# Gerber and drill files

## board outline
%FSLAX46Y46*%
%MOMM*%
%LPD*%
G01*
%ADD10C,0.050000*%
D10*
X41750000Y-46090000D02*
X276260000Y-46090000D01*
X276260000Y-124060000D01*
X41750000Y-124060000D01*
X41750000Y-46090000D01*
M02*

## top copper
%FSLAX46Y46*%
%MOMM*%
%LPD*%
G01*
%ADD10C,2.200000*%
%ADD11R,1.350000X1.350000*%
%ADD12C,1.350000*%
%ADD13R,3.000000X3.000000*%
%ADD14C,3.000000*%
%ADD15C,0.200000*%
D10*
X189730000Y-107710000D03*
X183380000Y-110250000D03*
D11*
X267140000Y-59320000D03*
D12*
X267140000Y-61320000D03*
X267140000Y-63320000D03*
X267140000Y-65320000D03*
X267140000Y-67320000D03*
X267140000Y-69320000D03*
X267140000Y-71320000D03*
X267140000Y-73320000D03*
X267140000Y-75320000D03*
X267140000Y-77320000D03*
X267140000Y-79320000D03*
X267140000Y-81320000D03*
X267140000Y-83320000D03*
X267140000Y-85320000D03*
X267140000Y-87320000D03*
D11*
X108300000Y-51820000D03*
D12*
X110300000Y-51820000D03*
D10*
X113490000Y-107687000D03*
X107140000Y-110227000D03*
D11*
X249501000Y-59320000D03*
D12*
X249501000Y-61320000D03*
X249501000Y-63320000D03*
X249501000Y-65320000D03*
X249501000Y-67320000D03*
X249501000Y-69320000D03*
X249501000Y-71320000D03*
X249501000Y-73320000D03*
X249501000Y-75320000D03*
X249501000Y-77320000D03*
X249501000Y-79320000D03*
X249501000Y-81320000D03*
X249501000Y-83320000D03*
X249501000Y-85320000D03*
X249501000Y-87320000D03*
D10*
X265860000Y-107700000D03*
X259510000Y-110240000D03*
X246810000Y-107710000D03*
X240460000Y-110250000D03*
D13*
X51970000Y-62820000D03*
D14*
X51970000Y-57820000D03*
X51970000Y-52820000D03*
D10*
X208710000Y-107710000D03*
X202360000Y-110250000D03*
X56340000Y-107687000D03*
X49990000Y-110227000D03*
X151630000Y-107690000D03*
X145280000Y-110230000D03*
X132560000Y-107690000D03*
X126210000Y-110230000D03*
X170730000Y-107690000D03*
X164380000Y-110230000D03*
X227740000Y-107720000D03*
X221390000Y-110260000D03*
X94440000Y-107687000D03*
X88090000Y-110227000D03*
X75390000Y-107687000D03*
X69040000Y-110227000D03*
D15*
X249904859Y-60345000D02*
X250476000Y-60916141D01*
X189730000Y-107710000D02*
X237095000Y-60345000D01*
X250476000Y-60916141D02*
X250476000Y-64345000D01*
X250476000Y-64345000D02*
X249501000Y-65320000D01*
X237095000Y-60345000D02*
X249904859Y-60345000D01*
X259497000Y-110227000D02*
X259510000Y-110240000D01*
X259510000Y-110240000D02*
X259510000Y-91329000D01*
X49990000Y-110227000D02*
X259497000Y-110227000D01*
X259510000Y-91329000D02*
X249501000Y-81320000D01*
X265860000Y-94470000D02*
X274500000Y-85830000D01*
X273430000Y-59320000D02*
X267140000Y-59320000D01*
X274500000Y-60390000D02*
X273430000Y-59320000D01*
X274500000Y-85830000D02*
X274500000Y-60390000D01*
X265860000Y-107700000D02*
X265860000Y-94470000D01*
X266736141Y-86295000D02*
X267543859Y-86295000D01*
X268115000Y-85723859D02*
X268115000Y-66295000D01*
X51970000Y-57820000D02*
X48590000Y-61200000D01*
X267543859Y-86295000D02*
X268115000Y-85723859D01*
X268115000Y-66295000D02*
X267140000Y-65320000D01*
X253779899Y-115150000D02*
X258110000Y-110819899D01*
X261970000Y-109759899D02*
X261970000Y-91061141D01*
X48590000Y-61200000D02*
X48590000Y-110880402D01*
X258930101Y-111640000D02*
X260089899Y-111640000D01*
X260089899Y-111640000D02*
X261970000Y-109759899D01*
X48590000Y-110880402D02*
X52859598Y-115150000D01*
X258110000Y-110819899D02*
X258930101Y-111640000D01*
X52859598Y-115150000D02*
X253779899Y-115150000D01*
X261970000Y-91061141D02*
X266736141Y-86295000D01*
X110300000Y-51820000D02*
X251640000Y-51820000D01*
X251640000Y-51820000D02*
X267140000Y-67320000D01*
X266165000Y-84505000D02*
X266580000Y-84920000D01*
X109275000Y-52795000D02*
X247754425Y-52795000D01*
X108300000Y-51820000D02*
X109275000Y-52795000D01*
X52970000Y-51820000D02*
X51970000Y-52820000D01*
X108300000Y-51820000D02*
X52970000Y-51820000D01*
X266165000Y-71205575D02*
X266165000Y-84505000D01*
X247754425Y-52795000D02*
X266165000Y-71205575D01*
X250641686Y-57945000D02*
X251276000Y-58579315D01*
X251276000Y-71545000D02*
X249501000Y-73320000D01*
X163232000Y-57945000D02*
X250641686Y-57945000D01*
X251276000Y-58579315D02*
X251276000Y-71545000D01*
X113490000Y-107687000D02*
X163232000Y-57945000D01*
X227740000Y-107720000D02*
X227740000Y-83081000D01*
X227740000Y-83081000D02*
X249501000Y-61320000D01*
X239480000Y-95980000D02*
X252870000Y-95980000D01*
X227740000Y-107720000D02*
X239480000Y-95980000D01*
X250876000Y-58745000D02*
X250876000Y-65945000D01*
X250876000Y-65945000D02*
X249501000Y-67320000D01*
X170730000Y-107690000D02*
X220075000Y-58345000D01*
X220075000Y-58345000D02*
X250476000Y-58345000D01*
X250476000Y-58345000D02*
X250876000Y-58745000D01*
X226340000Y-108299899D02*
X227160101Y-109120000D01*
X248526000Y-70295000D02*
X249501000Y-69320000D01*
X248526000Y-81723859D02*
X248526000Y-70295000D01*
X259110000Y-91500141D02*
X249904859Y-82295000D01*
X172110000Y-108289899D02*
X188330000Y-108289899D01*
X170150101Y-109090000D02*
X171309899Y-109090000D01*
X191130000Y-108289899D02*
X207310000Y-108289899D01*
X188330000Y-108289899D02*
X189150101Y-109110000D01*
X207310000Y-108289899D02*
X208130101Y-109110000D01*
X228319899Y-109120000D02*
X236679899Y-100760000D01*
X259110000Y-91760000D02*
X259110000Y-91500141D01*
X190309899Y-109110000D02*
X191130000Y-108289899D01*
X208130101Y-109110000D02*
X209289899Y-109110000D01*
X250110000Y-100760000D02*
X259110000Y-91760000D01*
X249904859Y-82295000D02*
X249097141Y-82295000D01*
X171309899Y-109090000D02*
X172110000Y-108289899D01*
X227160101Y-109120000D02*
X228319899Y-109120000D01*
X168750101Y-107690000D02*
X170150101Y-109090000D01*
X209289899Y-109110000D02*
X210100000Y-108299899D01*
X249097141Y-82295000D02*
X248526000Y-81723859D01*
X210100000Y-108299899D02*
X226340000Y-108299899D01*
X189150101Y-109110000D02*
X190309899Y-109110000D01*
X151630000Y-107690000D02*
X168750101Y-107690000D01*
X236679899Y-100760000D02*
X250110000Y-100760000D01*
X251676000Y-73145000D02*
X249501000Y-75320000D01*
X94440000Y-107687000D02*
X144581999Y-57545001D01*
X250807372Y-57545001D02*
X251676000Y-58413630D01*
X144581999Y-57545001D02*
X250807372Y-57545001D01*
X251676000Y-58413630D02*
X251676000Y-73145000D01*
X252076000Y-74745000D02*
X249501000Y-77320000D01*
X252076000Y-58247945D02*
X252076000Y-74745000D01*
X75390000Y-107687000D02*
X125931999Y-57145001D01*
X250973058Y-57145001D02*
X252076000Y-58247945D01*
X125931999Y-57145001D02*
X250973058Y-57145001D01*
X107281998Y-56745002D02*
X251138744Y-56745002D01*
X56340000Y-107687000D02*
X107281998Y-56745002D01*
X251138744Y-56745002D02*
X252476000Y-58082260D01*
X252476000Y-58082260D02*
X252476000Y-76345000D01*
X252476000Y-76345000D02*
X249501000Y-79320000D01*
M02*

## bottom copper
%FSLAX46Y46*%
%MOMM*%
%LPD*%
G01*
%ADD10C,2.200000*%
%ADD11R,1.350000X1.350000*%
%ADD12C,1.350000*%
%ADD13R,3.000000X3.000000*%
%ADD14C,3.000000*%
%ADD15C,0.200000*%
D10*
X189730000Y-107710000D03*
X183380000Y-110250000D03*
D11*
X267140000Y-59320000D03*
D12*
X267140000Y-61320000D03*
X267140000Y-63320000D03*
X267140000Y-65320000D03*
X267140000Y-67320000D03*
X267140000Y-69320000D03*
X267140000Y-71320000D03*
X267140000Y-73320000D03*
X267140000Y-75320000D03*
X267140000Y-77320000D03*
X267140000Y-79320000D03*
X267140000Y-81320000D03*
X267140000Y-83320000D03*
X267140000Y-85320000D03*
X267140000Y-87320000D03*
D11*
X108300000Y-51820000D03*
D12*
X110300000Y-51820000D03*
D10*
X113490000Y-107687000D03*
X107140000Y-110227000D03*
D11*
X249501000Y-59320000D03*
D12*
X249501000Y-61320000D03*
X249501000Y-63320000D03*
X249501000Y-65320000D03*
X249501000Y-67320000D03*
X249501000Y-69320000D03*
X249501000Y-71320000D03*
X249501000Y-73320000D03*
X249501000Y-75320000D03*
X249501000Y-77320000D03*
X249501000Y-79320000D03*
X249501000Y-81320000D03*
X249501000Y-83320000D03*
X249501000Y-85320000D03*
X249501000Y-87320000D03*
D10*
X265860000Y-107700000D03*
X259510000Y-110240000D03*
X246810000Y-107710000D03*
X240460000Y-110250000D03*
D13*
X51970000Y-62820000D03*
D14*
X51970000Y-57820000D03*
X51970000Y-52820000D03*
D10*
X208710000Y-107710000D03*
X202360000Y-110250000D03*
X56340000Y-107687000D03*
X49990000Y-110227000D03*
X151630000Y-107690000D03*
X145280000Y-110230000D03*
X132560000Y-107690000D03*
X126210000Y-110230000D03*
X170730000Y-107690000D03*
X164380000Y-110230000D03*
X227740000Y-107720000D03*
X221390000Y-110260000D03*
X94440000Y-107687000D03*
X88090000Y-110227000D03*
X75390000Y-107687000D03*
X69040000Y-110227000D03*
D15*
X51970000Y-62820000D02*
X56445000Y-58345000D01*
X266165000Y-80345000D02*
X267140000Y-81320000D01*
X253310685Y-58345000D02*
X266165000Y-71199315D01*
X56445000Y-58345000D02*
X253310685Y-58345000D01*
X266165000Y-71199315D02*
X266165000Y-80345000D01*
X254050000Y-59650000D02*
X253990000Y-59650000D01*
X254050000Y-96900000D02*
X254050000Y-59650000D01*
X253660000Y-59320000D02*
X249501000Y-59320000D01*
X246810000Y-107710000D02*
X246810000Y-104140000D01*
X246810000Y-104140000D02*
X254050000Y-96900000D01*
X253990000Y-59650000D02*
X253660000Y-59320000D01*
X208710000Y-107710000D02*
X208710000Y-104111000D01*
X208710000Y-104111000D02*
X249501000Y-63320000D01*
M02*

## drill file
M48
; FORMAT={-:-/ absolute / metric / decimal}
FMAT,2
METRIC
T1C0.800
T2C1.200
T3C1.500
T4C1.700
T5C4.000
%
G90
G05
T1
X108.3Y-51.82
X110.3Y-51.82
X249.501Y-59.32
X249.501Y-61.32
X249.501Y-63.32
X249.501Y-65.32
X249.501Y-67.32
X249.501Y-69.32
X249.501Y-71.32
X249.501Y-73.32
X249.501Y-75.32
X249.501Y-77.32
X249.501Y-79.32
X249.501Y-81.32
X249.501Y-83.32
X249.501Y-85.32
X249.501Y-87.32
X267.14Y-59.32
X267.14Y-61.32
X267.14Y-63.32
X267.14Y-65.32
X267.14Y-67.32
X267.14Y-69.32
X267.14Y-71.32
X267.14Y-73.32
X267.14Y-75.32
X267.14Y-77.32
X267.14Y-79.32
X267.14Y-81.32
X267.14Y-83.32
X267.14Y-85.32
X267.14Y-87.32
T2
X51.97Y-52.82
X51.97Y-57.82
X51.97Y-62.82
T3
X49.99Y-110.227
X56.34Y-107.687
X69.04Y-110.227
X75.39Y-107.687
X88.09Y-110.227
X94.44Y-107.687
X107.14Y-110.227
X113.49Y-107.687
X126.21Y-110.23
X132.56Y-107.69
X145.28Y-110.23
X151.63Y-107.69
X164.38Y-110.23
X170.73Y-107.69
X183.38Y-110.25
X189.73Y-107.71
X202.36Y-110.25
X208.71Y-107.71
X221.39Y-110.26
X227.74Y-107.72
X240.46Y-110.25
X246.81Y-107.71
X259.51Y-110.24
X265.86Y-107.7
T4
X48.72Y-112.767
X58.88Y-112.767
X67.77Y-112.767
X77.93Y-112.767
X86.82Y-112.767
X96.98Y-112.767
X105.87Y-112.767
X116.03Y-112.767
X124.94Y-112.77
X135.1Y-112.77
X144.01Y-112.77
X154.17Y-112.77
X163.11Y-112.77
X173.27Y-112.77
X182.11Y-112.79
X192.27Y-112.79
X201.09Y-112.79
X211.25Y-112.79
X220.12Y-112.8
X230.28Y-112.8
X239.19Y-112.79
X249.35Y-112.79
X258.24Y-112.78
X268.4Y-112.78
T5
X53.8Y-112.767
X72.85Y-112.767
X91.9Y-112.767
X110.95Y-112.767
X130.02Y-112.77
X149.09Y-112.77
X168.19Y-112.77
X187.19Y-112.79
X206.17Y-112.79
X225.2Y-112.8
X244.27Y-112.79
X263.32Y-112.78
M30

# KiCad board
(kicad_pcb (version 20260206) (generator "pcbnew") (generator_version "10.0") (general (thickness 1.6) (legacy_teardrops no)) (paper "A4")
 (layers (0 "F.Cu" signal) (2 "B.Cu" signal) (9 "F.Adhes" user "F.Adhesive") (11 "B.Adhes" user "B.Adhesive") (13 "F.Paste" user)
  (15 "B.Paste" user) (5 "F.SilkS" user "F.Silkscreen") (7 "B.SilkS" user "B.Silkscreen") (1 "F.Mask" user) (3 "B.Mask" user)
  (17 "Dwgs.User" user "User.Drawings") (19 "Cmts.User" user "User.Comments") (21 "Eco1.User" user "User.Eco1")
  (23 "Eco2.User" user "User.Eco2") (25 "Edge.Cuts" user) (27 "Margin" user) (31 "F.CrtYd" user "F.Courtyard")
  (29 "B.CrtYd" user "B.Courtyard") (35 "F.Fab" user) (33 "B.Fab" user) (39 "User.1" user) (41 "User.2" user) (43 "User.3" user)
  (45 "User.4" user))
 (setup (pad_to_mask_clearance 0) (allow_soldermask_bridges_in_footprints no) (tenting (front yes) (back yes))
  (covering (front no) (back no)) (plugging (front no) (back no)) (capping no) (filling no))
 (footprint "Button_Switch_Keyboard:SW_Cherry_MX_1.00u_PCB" (layer "F.Cu") (at 189.73 107.71)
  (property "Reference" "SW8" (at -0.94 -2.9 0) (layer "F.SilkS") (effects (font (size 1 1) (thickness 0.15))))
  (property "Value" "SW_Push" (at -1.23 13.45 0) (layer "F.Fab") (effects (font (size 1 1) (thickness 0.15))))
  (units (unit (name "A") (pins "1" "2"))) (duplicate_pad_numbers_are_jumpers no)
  (pad "" np_thru_hole circle (at -7.62 5.08) (size 1.7 1.7) (drill 1.7) (layers "*.Cu" "*.Mask"))
  (pad "" np_thru_hole circle (at -2.54 5.08) (size 4 4) (drill 4) (layers "*.Cu" "*.Mask"))
  (pad "" np_thru_hole circle (at 2.54 5.08) (size 1.7 1.7) (drill 1.7) (layers "*.Cu" "*.Mask"))
  (pad "1" thru_hole circle (at 0 0) (size 2.2 2.2) (drill 1.5) (layers "*.Cu" "*.Mask") (remove_unused_layers no) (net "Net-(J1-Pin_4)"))
  (pad "2" thru_hole circle (at -6.35 2.54) (size 2.2 2.2) (drill 1.5) (layers "*.Cu" "*.Mask") (remove_unused_layers no)
   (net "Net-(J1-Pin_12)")))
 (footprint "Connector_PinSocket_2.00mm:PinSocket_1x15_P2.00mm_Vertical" (layer "F.Cu") (at 267.14 59.32)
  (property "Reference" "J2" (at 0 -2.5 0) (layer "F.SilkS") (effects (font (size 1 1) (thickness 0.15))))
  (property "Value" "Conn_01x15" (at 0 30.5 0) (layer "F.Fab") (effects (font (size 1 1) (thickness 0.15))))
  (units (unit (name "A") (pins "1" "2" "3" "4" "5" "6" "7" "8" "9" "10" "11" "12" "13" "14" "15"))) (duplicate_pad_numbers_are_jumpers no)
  (pad "1" thru_hole rect (at 0 0) (size 1.35 1.35) (drill 0.8) (layers "*.Cu" "*.Mask") (remove_unused_layers no) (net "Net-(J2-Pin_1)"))
  (pad "2" thru_hole circle (at 0 2) (size 1.35 1.35) (drill 0.8) (layers "*.Cu" "*.Mask") (remove_unused_layers no)
   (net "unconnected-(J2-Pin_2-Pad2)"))
  (pad "3" thru_hole circle (at 0 4) (size 1.35 1.35) (drill 0.8) (layers "*.Cu" "*.Mask") (remove_unused_layers no)
   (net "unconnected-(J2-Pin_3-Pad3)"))
  (pad "4" thru_hole circle (at 0 6) (size 1.35 1.35) (drill 0.8) (layers "*.Cu" "*.Mask") (remove_unused_layers no) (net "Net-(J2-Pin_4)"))
  (pad "5" thru_hole circle (at 0 8) (size 1.35 1.35) (drill 0.8) (layers "*.Cu" "*.Mask") (remove_unused_layers no) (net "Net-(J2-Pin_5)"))
  (pad "6" thru_hole circle (at 0 10) (size 1.35 1.35) (drill 0.8) (layers "*.Cu" "*.Mask") (remove_unused_layers no)
   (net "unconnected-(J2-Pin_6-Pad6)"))
  (pad "7" thru_hole circle (at 0 12) (size 1.35 1.35) (drill 0.8) (layers "*.Cu" "*.Mask") (remove_unused_layers no)
   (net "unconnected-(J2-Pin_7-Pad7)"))
  (pad "8" thru_hole circle (at 0 14) (size 1.35 1.35) (drill 0.8) (layers "*.Cu" "*.Mask") (remove_unused_layers no)
   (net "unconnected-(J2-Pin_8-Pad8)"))
  (pad "9" thru_hole circle (at 0 16) (size 1.35 1.35) (drill 0.8) (layers "*.Cu" "*.Mask") (remove_unused_layers no)
   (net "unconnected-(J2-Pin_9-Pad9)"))
  (pad "10" thru_hole circle (at 0 18) (size 1.35 1.35) (drill 0.8) (layers "*.Cu" "*.Mask") (remove_unused_layers no)
   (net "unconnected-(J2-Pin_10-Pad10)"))
  (pad "11" thru_hole circle (at 0 20) (size 1.35 1.35) (drill 0.8) (layers "*.Cu" "*.Mask") (remove_unused_layers no)
   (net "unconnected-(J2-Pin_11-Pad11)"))
  (pad "12" thru_hole circle (at 0 22) (size 1.35 1.35) (drill 0.8) (layers "*.Cu" "*.Mask") (remove_unused_layers no)
   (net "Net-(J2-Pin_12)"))
  (pad "13" thru_hole circle (at 0 24) (size 1.35 1.35) (drill 0.8) (layers "*.Cu" "*.Mask") (remove_unused_layers no)
   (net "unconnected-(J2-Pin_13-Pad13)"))
  (pad "14" thru_hole circle (at 0 26) (size 1.35 1.35) (drill 0.8) (layers "*.Cu" "*.Mask") (remove_unused_layers no)
   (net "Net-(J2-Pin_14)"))
  (pad "15" thru_hole circle (at 0 28) (size 1.35 1.35) (drill 0.8) (layers "*.Cu" "*.Mask") (remove_unused_layers no)
   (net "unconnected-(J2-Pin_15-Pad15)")))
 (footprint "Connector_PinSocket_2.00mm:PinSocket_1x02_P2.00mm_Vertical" (layer "F.Cu") (at 108.3 51.82 90)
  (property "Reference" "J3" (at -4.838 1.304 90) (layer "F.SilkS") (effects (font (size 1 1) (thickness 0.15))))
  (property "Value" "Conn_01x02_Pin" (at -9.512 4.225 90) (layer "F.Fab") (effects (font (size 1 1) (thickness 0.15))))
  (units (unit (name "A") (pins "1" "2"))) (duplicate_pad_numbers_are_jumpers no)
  (pad "1" thru_hole rect (at 0 0 90) (size 1.35 1.35) (drill 0.8) (layers "*.Cu" "*.Mask") (remove_unused_layers no)
   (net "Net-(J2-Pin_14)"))
  (pad "2" thru_hole circle (at 0 2 90) (size 1.35 1.35) (drill 0.8) (layers "*.Cu" "*.Mask") (remove_unused_layers no)
   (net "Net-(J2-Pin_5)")))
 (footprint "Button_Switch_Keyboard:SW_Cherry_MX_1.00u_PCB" (layer "F.Cu") (at 113.49 107.687)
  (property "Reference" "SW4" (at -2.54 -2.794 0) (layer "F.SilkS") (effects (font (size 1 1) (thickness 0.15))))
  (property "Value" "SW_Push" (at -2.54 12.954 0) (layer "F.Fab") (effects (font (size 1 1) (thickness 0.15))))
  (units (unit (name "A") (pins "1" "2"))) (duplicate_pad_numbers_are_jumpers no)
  (pad "" np_thru_hole circle (at -7.62 5.08) (size 1.7 1.7) (drill 1.7) (layers "*.Cu" "*.Mask"))
  (pad "" np_thru_hole circle (at -2.54 5.08) (size 4 4) (drill 4) (layers "*.Cu" "*.Mask"))
  (pad "" np_thru_hole circle (at 2.54 5.08) (size 1.7 1.7) (drill 1.7) (layers "*.Cu" "*.Mask"))
  (pad "1" thru_hole circle (at 0 0) (size 2.2 2.2) (drill 1.5) (layers "*.Cu" "*.Mask") (remove_unused_layers no) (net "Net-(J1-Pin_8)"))
  (pad "2" thru_hole circle (at -6.35 2.54) (size 2.2 2.2) (drill 1.5) (layers "*.Cu" "*.Mask") (remove_unused_layers no)
   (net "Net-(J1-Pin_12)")))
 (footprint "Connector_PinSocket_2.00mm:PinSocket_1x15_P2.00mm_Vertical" (layer "F.Cu") (at 249.501 59.32)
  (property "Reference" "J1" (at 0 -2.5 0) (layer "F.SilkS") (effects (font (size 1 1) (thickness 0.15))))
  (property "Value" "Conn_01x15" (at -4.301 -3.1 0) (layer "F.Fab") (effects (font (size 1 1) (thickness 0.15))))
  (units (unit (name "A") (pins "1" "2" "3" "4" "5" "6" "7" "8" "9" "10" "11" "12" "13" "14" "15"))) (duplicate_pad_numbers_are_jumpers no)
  (pad "1" thru_hole rect (at 0 0) (size 1.35 1.35) (drill 0.8) (layers "*.Cu" "*.Mask") (remove_unused_layers no) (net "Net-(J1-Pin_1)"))
  (pad "2" thru_hole circle (at 0 2) (size 1.35 1.35) (drill 0.8) (layers "*.Cu" "*.Mask") (remove_unused_layers no) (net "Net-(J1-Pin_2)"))
  (pad "3" thru_hole circle (at 0 4) (size 1.35 1.35) (drill 0.8) (layers "*.Cu" "*.Mask") (remove_unused_layers no) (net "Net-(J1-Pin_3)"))
  (pad "4" thru_hole circle (at 0 6) (size 1.35 1.35) (drill 0.8) (layers "*.Cu" "*.Mask") (remove_unused_layers no) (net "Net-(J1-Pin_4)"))
  (pad "5" thru_hole circle (at 0 8) (size 1.35 1.35) (drill 0.8) (layers "*.Cu" "*.Mask") (remove_unused_layers no) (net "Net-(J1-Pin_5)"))
  (pad "6" thru_hole circle (at 0 10) (size 1.35 1.35) (drill 0.8) (layers "*.Cu" "*.Mask") (remove_unused_layers no) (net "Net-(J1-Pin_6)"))
  (pad "7" thru_hole circle (at 0 12) (size 1.35 1.35) (drill 0.8) (layers "*.Cu" "*.Mask") (remove_unused_layers no) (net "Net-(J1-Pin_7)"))
  (pad "8" thru_hole circle (at 0 14) (size 1.35 1.35) (drill 0.8) (layers "*.Cu" "*.Mask") (remove_unused_layers no) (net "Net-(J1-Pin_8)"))
  (pad "9" thru_hole circle (at 0 16) (size 1.35 1.35) (drill 0.8) (layers "*.Cu" "*.Mask") (remove_unused_layers no) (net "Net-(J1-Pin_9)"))
  (pad "10" thru_hole circle (at 0 18) (size 1.35 1.35) (drill 0.8) (layers "*.Cu" "*.Mask") (remove_unused_layers no)
   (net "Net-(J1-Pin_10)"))
  (pad "11" thru_hole circle (at 0 20) (size 1.35 1.35) (drill 0.8) (layers "*.Cu" "*.Mask") (remove_unused_layers no)
   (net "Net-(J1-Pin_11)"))
  (pad "12" thru_hole circle (at 0 22) (size 1.35 1.35) (drill 0.8) (layers "*.Cu" "*.Mask") (remove_unused_layers no)
   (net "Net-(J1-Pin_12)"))
  (pad "13" thru_hole circle (at 0 24) (size 1.35 1.35) (drill 0.8) (layers "*.Cu" "*.Mask") (remove_unused_layers no)
   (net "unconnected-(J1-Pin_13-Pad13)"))
  (pad "14" thru_hole circle (at 0 26) (size 1.35 1.35) (drill 0.8) (layers "*.Cu" "*.Mask") (remove_unused_layers no)
   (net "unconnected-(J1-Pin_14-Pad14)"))
  (pad "15" thru_hole circle (at 0 28) (size 1.35 1.35) (drill 0.8) (layers "*.Cu" "*.Mask") (remove_unused_layers no)
   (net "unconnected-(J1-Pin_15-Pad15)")))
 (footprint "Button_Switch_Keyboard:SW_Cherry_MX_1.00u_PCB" (layer "F.Cu") (at 265.86 107.7)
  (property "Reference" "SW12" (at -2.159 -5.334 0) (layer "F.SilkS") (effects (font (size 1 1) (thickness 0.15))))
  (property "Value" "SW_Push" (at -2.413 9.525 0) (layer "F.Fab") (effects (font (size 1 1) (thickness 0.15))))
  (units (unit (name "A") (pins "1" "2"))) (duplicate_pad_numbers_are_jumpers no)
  (pad "" np_thru_hole circle (at -7.62 5.08) (size 1.7 1.7) (drill 1.7) (layers "*.Cu" "*.Mask"))
  (pad "" np_thru_hole circle (at -2.54 5.08) (size 4 4) (drill 4) (layers "*.Cu" "*.Mask"))
  (pad "" np_thru_hole circle (at 2.54 5.08) (size 1.7 1.7) (drill 1.7) (layers "*.Cu" "*.Mask"))
  (pad "1" thru_hole circle (at 0 0) (size 2.2 2.2) (drill 1.5) (layers "*.Cu" "*.Mask") (remove_unused_layers no) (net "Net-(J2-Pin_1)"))
  (pad "2" thru_hole circle (at -6.35 2.54) (size 2.2 2.2) (drill 1.5) (layers "*.Cu" "*.Mask") (remove_unused_layers no)
   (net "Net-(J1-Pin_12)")))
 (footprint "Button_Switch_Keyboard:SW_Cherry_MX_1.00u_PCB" (layer "F.Cu") (at 246.81 107.71)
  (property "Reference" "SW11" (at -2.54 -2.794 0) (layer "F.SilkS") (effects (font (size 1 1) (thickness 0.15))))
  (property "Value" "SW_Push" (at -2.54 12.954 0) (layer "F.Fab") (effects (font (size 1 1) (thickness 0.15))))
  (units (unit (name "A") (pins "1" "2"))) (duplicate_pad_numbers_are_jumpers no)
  (pad "" np_thru_hole circle (at -7.62 5.08) (size 1.7 1.7) (drill 1.7) (layers "*.Cu" "*.Mask"))
  (pad "" np_thru_hole circle (at -2.54 5.08) (size 4 4) (drill 4) (layers "*.Cu" "*.Mask"))
  (pad "" np_thru_hole circle (at 2.54 5.08) (size 1.7 1.7) (drill 1.7) (layers "*.Cu" "*.Mask"))
  (pad "1" thru_hole circle (at 0 0) (size 2.2 2.2) (drill 1.5) (layers "*.Cu" "*.Mask") (remove_unused_layers no) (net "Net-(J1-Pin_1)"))
  (pad "2" thru_hole circle (at -6.35 2.54) (size 2.2 2.2) (drill 1.5) (layers "*.Cu" "*.Mask") (remove_unused_layers no)
   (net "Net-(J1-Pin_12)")))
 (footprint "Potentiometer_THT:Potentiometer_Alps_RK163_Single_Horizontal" (layer "F.Cu") (at 51.97 62.82 180)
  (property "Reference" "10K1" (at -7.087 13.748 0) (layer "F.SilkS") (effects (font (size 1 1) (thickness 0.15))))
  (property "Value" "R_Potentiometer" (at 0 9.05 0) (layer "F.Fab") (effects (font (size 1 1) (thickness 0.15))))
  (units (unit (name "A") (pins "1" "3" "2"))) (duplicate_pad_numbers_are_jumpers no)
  (pad "1" thru_hole rect (at 0 0) (size 3 3) (drill 1.2) (layers "*.Cu" "*.Mask") (remove_unused_layers no) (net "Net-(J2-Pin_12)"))
  (pad "2" thru_hole circle (at 0 5) (size 3 3) (drill 1.2) (layers "*.Cu" "*.Mask") (remove_unused_layers no) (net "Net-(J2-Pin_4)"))
  (pad "3" thru_hole circle (at 0 10) (size 3 3) (drill 1.2) (layers "*.Cu" "*.Mask") (remove_unused_layers no) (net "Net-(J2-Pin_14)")))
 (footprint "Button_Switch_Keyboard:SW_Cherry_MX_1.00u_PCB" (layer "F.Cu") (at 208.71 107.71)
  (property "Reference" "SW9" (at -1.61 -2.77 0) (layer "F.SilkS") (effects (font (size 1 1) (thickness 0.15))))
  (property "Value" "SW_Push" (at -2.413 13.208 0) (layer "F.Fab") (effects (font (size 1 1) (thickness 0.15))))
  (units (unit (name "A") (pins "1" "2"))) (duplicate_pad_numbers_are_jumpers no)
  (pad "" np_thru_hole circle (at -7.62 5.08) (size 1.7 1.7) (drill 1.7) (layers "*.Cu" "*.Mask"))
  (pad "" np_thru_hole circle (at -2.54 5.08) (size 4 4) (drill 4) (layers "*.Cu" "*.Mask"))
  (pad "" np_thru_hole circle (at 2.54 5.08) (size 1.7 1.7) (drill 1.7) (layers "*.Cu" "*.Mask"))
  (pad "1" thru_hole circle (at 0 0) (size 2.2 2.2) (drill 1.5) (layers "*.Cu" "*.Mask") (remove_unused_layers no) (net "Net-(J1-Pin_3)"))
  (pad "2" thru_hole circle (at -6.35 2.54) (size 2.2 2.2) (drill 1.5) (layers "*.Cu" "*.Mask") (remove_unused_layers no)
   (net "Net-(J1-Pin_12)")))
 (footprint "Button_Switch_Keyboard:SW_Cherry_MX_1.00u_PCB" (layer "F.Cu") (at 56.34 107.687)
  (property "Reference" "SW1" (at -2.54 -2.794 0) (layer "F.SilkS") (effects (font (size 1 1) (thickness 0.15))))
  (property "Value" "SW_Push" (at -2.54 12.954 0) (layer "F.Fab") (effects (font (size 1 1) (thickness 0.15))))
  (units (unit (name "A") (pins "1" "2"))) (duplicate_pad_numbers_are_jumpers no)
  (pad "" np_thru_hole circle (at -7.62 5.08) (size 1.7 1.7) (drill 1.7) (layers "*.Cu" "*.Mask"))
  (pad "" np_thru_hole circle (at -2.54 5.08) (size 4 4) (drill 4) (layers "*.Cu" "*.Mask"))
  (pad "" np_thru_hole circle (at 2.54 5.08) (size 1.7 1.7) (drill 1.7) (layers "*.Cu" "*.Mask"))
  (pad "1" thru_hole circle (at 0 0) (size 2.2 2.2) (drill 1.5) (layers "*.Cu" "*.Mask") (remove_unused_layers no) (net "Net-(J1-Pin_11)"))
  (pad "2" thru_hole circle (at -6.35 2.54) (size 2.2 2.2) (drill 1.5) (layers "*.Cu" "*.Mask") (remove_unused_layers no)
   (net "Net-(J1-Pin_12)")))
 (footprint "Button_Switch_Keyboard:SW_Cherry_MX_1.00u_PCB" (layer "F.Cu") (at 151.63 107.69)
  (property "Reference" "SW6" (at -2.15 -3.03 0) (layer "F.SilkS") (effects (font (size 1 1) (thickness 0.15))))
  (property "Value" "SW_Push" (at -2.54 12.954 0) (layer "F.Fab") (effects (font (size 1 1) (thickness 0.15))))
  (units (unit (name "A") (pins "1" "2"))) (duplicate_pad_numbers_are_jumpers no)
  (pad "" np_thru_hole circle (at -7.62 5.08) (size 1.7 1.7) (drill 1.7) (layers "*.Cu" "*.Mask"))
  (pad "" np_thru_hole circle (at -2.54 5.08) (size 4 4) (drill 4) (layers "*.Cu" "*.Mask"))
  (pad "" np_thru_hole circle (at 2.54 5.08) (size 1.7 1.7) (drill 1.7) (layers "*.Cu" "*.Mask"))
  (pad "1" thru_hole circle (at 0 0) (size 2.2 2.2) (drill 1.5) (layers "*.Cu" "*.Mask") (remove_unused_layers no) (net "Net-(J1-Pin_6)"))
  (pad "2" thru_hole circle (at -6.35 2.54) (size 2.2 2.2) (drill 1.5) (layers "*.Cu" "*.Mask") (remove_unused_layers no)
   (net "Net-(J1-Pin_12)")))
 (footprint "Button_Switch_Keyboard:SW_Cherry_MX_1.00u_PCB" (layer "F.Cu") (at 132.56 107.69)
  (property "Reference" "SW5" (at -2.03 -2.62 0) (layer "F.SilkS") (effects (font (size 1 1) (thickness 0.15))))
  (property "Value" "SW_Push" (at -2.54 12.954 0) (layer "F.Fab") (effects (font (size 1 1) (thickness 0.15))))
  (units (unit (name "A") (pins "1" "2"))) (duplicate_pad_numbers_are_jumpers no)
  (pad "" np_thru_hole circle (at -7.62 5.08) (size 1.7 1.7) (drill 1.7) (layers "*.Cu" "*.Mask"))
  (pad "" np_thru_hole circle (at -2.54 5.08) (size 4 4) (drill 4) (layers "*.Cu" "*.Mask"))
  (pad "" np_thru_hole circle (at 2.54 5.08) (size 1.7 1.7) (drill 1.7) (layers "*.Cu" "*.Mask"))
  (pad "1" thru_hole circle (at 0 0) (size 2.2 2.2) (drill 1.5) (layers "*.Cu" "*.Mask") (remove_unused_layers no) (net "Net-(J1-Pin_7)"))
  (pad "2" thru_hole circle (at -6.35 2.54) (size 2.2 2.2) (drill 1.5) (layers "*.Cu" "*.Mask") (remove_unused_layers no)
   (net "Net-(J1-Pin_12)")))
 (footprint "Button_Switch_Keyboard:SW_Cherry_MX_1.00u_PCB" (layer "F.Cu") (at 170.73 107.69)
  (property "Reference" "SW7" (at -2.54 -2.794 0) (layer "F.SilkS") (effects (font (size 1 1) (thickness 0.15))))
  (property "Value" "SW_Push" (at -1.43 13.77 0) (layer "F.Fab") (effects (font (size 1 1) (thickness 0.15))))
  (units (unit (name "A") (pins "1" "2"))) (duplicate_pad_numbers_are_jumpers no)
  (pad "" np_thru_hole circle (at -7.62 5.08) (size 1.7 1.7) (drill 1.7) (layers "*.Cu" "*.Mask"))
  (pad "" np_thru_hole circle (at -2.54 5.08) (size 4 4) (drill 4) (layers "*.Cu" "*.Mask"))
  (pad "" np_thru_hole circle (at 2.54 5.08) (size 1.7 1.7) (drill 1.7) (layers "*.Cu" "*.Mask"))
  (pad "1" thru_hole circle (at 0 0) (size 2.2 2.2) (drill 1.5) (layers "*.Cu" "*.Mask") (remove_unused_layers no) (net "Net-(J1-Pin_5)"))
  (pad "2" thru_hole circle (at -6.35 2.54) (size 2.2 2.2) (drill 1.5) (layers "*.Cu" "*.Mask") (remove_unused_layers no)
   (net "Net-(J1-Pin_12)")))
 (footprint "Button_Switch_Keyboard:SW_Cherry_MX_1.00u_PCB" (layer "F.Cu") (at 227.74 107.72)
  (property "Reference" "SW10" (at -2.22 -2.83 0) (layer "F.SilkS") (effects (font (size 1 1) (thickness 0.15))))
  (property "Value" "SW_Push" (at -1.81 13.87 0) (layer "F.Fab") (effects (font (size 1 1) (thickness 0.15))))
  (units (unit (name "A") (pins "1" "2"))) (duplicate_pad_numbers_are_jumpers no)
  (pad "" np_thru_hole circle (at -7.62 5.08) (size 1.7 1.7) (drill 1.7) (layers "*.Cu" "*.Mask"))
  (pad "" np_thru_hole circle (at -2.54 5.08) (size 4 4) (drill 4) (layers "*.Cu" "*.Mask"))
  (pad "" np_thru_hole circle (at 2.54 5.08) (size 1.7 1.7) (drill 1.7) (layers "*.Cu" "*.Mask"))
  (pad "1" thru_hole circle (at 0 0) (size 2.2 2.2) (drill 1.5) (layers "*.Cu" "*.Mask") (remove_unused_layers no) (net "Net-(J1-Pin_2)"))
  (pad "2" thru_hole circle (at -6.35 2.54) (size 2.2 2.2) (drill 1.5) (layers "*.Cu" "*.Mask") (remove_unused_layers no)
   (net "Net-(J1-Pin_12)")))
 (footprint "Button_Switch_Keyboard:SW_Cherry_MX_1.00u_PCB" (layer "F.Cu") (at 94.44 107.687)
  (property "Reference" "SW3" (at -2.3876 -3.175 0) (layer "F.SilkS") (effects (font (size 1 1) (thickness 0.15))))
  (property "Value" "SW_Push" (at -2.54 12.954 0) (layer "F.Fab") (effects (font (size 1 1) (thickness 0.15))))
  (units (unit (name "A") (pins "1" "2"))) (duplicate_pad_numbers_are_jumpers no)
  (pad "" np_thru_hole circle (at -7.62 5.08) (size 1.7 1.7) (drill 1.7) (layers "*.Cu" "*.Mask"))
  (pad "" np_thru_hole circle (at -2.54 5.08) (size 4 4) (drill 4) (layers "*.Cu" "*.Mask"))
  (pad "" np_thru_hole circle (at 2.54 5.08) (size 1.7 1.7) (drill 1.7) (layers "*.Cu" "*.Mask"))
  (pad "1" thru_hole circle (at 0 0) (size 2.2 2.2) (drill 1.5) (layers "*.Cu" "*.Mask") (remove_unused_layers no) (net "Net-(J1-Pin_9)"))
  (pad "2" thru_hole circle (at -6.35 2.54) (size 2.2 2.2) (drill 1.5) (layers "*.Cu" "*.Mask") (remove_unused_layers no)
   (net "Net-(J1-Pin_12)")))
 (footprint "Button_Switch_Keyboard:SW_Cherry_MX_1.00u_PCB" (layer "F.Cu") (at 75.39 107.687)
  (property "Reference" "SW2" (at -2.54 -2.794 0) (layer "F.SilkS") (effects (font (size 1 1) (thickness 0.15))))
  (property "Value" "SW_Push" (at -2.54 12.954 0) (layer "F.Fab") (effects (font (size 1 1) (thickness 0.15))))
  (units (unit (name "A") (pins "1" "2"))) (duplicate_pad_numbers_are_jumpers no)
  (pad "" np_thru_hole circle (at -7.62 5.08) (size 1.7 1.7) (drill 1.7) (layers "*.Cu" "*.Mask"))
  (pad "" np_thru_hole circle (at -2.54 5.08) (size 4 4) (drill 4) (layers "*.Cu" "*.Mask"))
  (pad "" np_thru_hole circle (at 2.54 5.08) (size 1.7 1.7) (drill 1.7) (layers "*.Cu" "*.Mask"))
  (pad "1" thru_hole circle (at 0 0) (size 2.2 2.2) (drill 1.5) (layers "*.Cu" "*.Mask") (remove_unused_layers no) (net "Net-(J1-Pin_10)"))
  (pad "2" thru_hole circle (at -6.35 2.54) (size 2.2 2.2) (drill 1.5) (layers "*.Cu" "*.Mask") (remove_unused_layers no)
   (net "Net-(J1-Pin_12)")))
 (gr_rect (start 41.75 46.09) (end 276.26 124.06) (stroke (width 0.05) (type default)) (fill no) (layer "Edge.Cuts"))
 (segment (start 249.904859 60.345) (end 250.476 60.916141) (width 0.2) (layer "F.Cu") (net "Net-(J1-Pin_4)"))
 (segment (start 189.73 107.71) (end 237.095 60.345) (width 0.2) (layer "F.Cu") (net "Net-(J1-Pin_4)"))
 (segment (start 250.476 60.916141) (end 250.476 64.345) (width 0.2) (layer "F.Cu") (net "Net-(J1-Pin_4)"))
 (segment (start 250.476 64.345) (end 249.501 65.32) (width 0.2) (layer "F.Cu") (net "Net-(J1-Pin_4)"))
 (segment (start 237.095 60.345) (end 249.904859 60.345) (width 0.2) (layer "F.Cu") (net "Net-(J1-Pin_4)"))
 (segment (start 259.497 110.227) (end 259.51 110.24) (width 0.2) (layer "F.Cu") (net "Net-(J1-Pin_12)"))
 (segment (start 259.51 110.24) (end 259.51 91.329) (width 0.2) (layer "F.Cu") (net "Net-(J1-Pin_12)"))
 (segment (start 49.99 110.227) (end 259.497 110.227) (width 0.2) (layer "F.Cu") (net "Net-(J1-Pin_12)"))
 (segment (start 259.51 91.329) (end 249.501 81.32) (width 0.2) (layer "F.Cu") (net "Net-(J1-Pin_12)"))
 (segment (start 265.86 94.47) (end 274.5 85.83) (width 0.2) (layer "F.Cu") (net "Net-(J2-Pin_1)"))
 (segment (start 273.43 59.32) (end 267.14 59.32) (width 0.2) (layer "F.Cu") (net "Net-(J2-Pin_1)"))
 (segment (start 274.5 60.39) (end 273.43 59.32) (width 0.2) (layer "F.Cu") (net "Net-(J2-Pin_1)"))
 (segment (start 274.5 85.83) (end 274.5 60.39) (width 0.2) (layer "F.Cu") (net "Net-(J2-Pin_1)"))
 (segment (start 265.86 107.7) (end 265.86 94.47) (width 0.2) (layer "F.Cu") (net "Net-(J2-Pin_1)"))
 (segment (start 266.736141 86.295) (end 267.543859 86.295) (width 0.2) (layer "F.Cu") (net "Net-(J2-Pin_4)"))
 (segment (start 268.115 85.723859) (end 268.115 66.295) (width 0.2) (layer "F.Cu") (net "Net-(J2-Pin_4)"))
 (segment (start 51.97 57.82) (end 48.59 61.2) (width 0.2) (layer "F.Cu") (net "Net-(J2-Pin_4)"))
 (segment (start 267.543859 86.295) (end 268.115 85.723859) (width 0.2) (layer "F.Cu") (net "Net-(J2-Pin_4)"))
 (segment (start 268.115 66.295) (end 267.14 65.32) (width 0.2) (layer "F.Cu") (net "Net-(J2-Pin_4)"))
 (segment (start 253.779899 115.15) (end 258.11 110.819899) (width 0.2) (layer "F.Cu") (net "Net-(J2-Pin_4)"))
 (segment (start 261.97 109.759899) (end 261.97 91.061141) (width 0.2) (layer "F.Cu") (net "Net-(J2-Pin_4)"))
 (segment (start 48.59 61.2) (end 48.59 110.880402) (width 0.2) (layer "F.Cu") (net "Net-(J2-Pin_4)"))
 (segment (start 258.930101 111.64) (end 260.089899 111.64) (width 0.2) (layer "F.Cu") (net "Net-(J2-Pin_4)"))
 (segment (start 260.089899 111.64) (end 261.97 109.759899) (width 0.2) (layer "F.Cu") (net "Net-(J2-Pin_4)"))
 (segment (start 48.59 110.880402) (end 52.859598 115.15) (width 0.2) (layer "F.Cu") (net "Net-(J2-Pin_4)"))
 (segment (start 258.11 110.819899) (end 258.930101 111.64) (width 0.2) (layer "F.Cu") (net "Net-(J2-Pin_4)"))
 (segment (start 52.859598 115.15) (end 253.779899 115.15) (width 0.2) (layer "F.Cu") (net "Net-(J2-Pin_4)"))
 (segment (start 261.97 91.061141) (end 266.736141 86.295) (width 0.2) (layer "F.Cu") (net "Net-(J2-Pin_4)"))
 (segment (start 110.3 51.82) (end 251.64 51.82) (width 0.2) (layer "F.Cu") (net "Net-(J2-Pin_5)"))
 (segment (start 251.64 51.82) (end 267.14 67.32) (width 0.2) (layer "F.Cu") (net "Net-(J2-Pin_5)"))
 (segment (start 51.97 62.82) (end 56.445 58.345) (width 0.2) (layer "B.Cu") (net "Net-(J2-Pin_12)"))
 (segment (start 266.165 80.345) (end 267.14 81.32) (width 0.2) (layer "B.Cu") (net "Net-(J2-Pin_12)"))
 (segment (start 253.310685 58.345) (end 266.165 71.199315) (width 0.2) (layer "B.Cu") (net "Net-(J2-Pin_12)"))
 (segment (start 56.445 58.345) (end 253.310685 58.345) (width 0.2) (layer "B.Cu") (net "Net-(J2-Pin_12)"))
 (segment (start 266.165 71.199315) (end 266.165 80.345) (width 0.2) (layer "B.Cu") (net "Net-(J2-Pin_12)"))
 (segment (start 266.165 84.505) (end 266.58 84.92) (width 0.2) (layer "F.Cu") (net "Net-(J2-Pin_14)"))
 (segment (start 109.275 52.795) (end 247.754425 52.795) (width 0.2) (layer "F.Cu") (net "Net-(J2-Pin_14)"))
 (segment (start 108.3 51.82) (end 109.275 52.795) (width 0.2) (layer "F.Cu") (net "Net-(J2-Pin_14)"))
 (segment (start 52.97 51.82) (end 51.97 52.82) (width 0.2) (layer "F.Cu") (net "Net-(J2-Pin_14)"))
 (segment (start 108.3 51.82) (end 52.97 51.82) (width 0.2) (layer "F.Cu") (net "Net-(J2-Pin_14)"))
 (segment (start 266.165 71.205575) (end 266.165 84.505) (width 0.2) (layer "F.Cu") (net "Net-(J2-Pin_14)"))
 (segment (start 247.754425 52.795) (end 266.165 71.205575) (width 0.2) (layer "F.Cu") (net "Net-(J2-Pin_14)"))
 (segment (start 250.641686 57.945) (end 251.276 58.579315) (width 0.2) (layer "F.Cu") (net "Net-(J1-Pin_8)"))
 (segment (start 251.276 71.545) (end 249.501 73.32) (width 0.2) (layer "F.Cu") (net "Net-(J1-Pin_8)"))
 (segment (start 163.232 57.945) (end 250.641686 57.945) (width 0.2) (layer "F.Cu") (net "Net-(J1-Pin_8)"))
 (segment (start 251.276 58.579315) (end 251.276 71.545) (width 0.2) (layer "F.Cu") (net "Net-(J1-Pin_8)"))
 (segment (start 113.49 107.687) (end 163.232 57.945) (width 0.2) (layer "F.Cu") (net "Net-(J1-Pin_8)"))
 (segment (start 254.05 59.65) (end 253.99 59.65) (width 0.2) (layer "B.Cu") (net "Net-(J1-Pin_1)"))
 (segment (start 254.05 96.9) (end 254.05 59.65) (width 0.2) (layer "B.Cu") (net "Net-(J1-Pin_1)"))
 (segment (start 253.66 59.32) (end 249.501 59.32) (width 0.2) (layer "B.Cu") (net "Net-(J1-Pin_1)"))
 (segment (start 246.81 107.71) (end 246.81 104.14) (width 0.2) (layer "B.Cu") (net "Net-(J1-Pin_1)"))
 (segment (start 246.81 104.14) (end 254.05 96.9) (width 0.2) (layer "B.Cu") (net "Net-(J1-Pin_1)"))
 (segment (start 253.99 59.65) (end 253.66 59.32) (width 0.2) (layer "B.Cu") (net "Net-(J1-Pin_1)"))
 (segment (start 227.74 107.72) (end 227.74 83.081) (width 0.2) (layer "F.Cu") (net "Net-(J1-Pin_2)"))
 (segment (start 227.74 83.081) (end 249.501 61.32) (width 0.2) (layer "F.Cu") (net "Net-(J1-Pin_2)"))
 (segment (start 239.48 95.98) (end 252.87 95.98) (width 0.2) (layer "F.Cu") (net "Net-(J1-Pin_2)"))
 (segment (start 227.74 107.72) (end 239.48 95.98) (width 0.2) (layer "F.Cu") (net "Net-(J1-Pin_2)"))
 (segment (start 208.71 107.71) (end 208.71 104.111) (width 0.2) (layer "B.Cu") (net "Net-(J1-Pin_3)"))
 (segment (start 208.71 104.111) (end 249.501 63.32) (width 0.2) (layer "B.Cu") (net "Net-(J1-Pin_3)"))
 (segment (start 250.876 58.745) (end 250.876 65.945) (width 0.2) (layer "F.Cu") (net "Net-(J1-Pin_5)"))
 (segment (start 250.876 65.945) (end 249.501 67.32) (width 0.2) (layer "F.Cu") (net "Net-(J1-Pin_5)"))
 (segment (start 170.73 107.69) (end 220.075 58.345) (width 0.2) (layer "F.Cu") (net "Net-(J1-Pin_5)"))
 (segment (start 220.075 58.345) (end 250.476 58.345) (width 0.2) (layer "F.Cu") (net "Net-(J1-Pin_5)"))
 (segment (start 250.476 58.345) (end 250.876 58.745) (width 0.2) (layer "F.Cu") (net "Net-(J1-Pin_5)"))
 (segment (start 226.34 108.299899) (end 227.160101 109.12) (width 0.2) (layer "F.Cu") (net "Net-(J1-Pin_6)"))
 (segment (start 248.526 70.295) (end 249.501 69.32) (width 0.2) (layer "F.Cu") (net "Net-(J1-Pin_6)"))
 (segment (start 248.526 81.723859) (end 248.526 70.295) (width 0.2) (layer "F.Cu") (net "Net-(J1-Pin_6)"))
 (segment (start 259.11 91.500141) (end 249.904859 82.295) (width 0.2) (layer "F.Cu") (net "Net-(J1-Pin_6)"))
 (segment (start 172.11 108.289899) (end 188.33 108.289899) (width 0.2) (layer "F.Cu") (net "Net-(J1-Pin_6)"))
 (segment (start 170.150101 109.09) (end 171.309899 109.09) (width 0.2) (layer "F.Cu") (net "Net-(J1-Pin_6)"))
 (segment (start 191.13 108.289899) (end 207.31 108.289899) (width 0.2) (layer "F.Cu") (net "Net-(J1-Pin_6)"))
 (segment (start 188.33 108.289899) (end 189.150101 109.11) (width 0.2) (layer "F.Cu") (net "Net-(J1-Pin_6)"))
 (segment (start 207.31 108.289899) (end 208.130101 109.11) (width 0.2) (layer "F.Cu") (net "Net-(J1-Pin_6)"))
 (segment (start 228.319899 109.12) (end 236.679899 100.76) (width 0.2) (layer "F.Cu") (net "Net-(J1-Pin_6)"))
 (segment (start 259.11 91.76) (end 259.11 91.500141) (width 0.2) (layer "F.Cu") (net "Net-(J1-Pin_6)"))
 (segment (start 190.309899 109.11) (end 191.13 108.289899) (width 0.2) (layer "F.Cu") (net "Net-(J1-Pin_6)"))
 (segment (start 208.130101 109.11) (end 209.289899 109.11) (width 0.2) (layer "F.Cu") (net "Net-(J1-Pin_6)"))
 (segment (start 250.11 100.76) (end 259.11 91.76) (width 0.2) (layer "F.Cu") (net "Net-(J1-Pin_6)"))
 (segment (start 249.904859 82.295) (end 249.097141 82.295) (width 0.2) (layer "F.Cu") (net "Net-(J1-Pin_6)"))
 (segment (start 171.309899 109.09) (end 172.11 108.289899) (width 0.2) (layer "F.Cu") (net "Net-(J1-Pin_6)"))
 (segment (start 227.160101 109.12) (end 228.319899 109.12) (width 0.2) (layer "F.Cu") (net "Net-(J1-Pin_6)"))
 (segment (start 168.750101 107.69) (end 170.150101 109.09) (width 0.2) (layer "F.Cu") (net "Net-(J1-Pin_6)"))
 (segment (start 209.289899 109.11) (end 210.1 108.299899) (width 0.2) (layer "F.Cu") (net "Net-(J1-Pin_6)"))
 (segment (start 249.097141 82.295) (end 248.526 81.723859) (width 0.2) (layer "F.Cu") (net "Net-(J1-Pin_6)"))
 (segment (start 210.1 108.299899) (end 226.34 108.299899) (width 0.2) (layer "F.Cu") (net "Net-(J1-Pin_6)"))
 (segment (start 189.150101 109.11) (end 190.309899 109.11) (width 0.2) (layer "F.Cu") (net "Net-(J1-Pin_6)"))
 (segment (start 151.63 107.69) (end 168.750101 107.69) (width 0.2) (layer "F.Cu") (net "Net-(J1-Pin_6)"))
 (segment (start 236.679899 100.76) (end 250.11 100.76) (width 0.2) (layer "F.Cu") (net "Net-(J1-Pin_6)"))
 (segment (start 251.676 73.145) (end 249.501 75.32) (width 0.2) (layer "F.Cu") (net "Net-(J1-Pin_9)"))
 (segment (start 94.44 107.687) (end 144.581999 57.545001) (width 0.2) (layer "F.Cu") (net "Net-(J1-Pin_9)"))
 (segment (start 250.807372 57.545001) (end 251.676 58.41363) (width 0.2) (layer "F.Cu") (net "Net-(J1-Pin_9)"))
 (segment (start 144.581999 57.545001) (end 250.807372 57.545001) (width 0.2) (layer "F.Cu") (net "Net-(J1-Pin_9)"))
 (segment (start 251.676 58.41363) (end 251.676 73.145) (width 0.2) (layer "F.Cu") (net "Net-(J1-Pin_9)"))
 (segment (start 252.076 74.745) (end 249.501 77.32) (width 0.2) (layer "F.Cu") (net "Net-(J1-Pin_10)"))
 (segment (start 252.076 58.247945) (end 252.076 74.745) (width 0.2) (layer "F.Cu") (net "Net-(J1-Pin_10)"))
 (segment (start 75.39 107.687) (end 125.931999 57.145001) (width 0.2) (layer "F.Cu") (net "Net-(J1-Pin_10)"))
 (segment (start 250.973058 57.145001) (end 252.076 58.247945) (width 0.2) (layer "F.Cu") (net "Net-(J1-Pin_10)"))
 (segment (start 125.931999 57.145001) (end 250.973058 57.145001) (width 0.2) (layer "F.Cu") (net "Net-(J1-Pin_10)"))
 (segment (start 107.281998 56.745002) (end 251.138744 56.745002) (width 0.2) (layer "F.Cu") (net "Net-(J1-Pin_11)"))
 (segment (start 56.34 107.687) (end 107.281998 56.745002) (width 0.2) (layer "F.Cu") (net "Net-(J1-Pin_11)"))
 (segment (start 251.138744 56.745002) (end 252.476 58.08226) (width 0.2) (layer "F.Cu") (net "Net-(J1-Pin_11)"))
 (segment (start 252.476 58.08226) (end 252.476 76.345) (width 0.2) (layer "F.Cu") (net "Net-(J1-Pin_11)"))
 (segment (start 252.476 76.345) (end 249.501 79.32) (width 0.2) (layer "F.Cu") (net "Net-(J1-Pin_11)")))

